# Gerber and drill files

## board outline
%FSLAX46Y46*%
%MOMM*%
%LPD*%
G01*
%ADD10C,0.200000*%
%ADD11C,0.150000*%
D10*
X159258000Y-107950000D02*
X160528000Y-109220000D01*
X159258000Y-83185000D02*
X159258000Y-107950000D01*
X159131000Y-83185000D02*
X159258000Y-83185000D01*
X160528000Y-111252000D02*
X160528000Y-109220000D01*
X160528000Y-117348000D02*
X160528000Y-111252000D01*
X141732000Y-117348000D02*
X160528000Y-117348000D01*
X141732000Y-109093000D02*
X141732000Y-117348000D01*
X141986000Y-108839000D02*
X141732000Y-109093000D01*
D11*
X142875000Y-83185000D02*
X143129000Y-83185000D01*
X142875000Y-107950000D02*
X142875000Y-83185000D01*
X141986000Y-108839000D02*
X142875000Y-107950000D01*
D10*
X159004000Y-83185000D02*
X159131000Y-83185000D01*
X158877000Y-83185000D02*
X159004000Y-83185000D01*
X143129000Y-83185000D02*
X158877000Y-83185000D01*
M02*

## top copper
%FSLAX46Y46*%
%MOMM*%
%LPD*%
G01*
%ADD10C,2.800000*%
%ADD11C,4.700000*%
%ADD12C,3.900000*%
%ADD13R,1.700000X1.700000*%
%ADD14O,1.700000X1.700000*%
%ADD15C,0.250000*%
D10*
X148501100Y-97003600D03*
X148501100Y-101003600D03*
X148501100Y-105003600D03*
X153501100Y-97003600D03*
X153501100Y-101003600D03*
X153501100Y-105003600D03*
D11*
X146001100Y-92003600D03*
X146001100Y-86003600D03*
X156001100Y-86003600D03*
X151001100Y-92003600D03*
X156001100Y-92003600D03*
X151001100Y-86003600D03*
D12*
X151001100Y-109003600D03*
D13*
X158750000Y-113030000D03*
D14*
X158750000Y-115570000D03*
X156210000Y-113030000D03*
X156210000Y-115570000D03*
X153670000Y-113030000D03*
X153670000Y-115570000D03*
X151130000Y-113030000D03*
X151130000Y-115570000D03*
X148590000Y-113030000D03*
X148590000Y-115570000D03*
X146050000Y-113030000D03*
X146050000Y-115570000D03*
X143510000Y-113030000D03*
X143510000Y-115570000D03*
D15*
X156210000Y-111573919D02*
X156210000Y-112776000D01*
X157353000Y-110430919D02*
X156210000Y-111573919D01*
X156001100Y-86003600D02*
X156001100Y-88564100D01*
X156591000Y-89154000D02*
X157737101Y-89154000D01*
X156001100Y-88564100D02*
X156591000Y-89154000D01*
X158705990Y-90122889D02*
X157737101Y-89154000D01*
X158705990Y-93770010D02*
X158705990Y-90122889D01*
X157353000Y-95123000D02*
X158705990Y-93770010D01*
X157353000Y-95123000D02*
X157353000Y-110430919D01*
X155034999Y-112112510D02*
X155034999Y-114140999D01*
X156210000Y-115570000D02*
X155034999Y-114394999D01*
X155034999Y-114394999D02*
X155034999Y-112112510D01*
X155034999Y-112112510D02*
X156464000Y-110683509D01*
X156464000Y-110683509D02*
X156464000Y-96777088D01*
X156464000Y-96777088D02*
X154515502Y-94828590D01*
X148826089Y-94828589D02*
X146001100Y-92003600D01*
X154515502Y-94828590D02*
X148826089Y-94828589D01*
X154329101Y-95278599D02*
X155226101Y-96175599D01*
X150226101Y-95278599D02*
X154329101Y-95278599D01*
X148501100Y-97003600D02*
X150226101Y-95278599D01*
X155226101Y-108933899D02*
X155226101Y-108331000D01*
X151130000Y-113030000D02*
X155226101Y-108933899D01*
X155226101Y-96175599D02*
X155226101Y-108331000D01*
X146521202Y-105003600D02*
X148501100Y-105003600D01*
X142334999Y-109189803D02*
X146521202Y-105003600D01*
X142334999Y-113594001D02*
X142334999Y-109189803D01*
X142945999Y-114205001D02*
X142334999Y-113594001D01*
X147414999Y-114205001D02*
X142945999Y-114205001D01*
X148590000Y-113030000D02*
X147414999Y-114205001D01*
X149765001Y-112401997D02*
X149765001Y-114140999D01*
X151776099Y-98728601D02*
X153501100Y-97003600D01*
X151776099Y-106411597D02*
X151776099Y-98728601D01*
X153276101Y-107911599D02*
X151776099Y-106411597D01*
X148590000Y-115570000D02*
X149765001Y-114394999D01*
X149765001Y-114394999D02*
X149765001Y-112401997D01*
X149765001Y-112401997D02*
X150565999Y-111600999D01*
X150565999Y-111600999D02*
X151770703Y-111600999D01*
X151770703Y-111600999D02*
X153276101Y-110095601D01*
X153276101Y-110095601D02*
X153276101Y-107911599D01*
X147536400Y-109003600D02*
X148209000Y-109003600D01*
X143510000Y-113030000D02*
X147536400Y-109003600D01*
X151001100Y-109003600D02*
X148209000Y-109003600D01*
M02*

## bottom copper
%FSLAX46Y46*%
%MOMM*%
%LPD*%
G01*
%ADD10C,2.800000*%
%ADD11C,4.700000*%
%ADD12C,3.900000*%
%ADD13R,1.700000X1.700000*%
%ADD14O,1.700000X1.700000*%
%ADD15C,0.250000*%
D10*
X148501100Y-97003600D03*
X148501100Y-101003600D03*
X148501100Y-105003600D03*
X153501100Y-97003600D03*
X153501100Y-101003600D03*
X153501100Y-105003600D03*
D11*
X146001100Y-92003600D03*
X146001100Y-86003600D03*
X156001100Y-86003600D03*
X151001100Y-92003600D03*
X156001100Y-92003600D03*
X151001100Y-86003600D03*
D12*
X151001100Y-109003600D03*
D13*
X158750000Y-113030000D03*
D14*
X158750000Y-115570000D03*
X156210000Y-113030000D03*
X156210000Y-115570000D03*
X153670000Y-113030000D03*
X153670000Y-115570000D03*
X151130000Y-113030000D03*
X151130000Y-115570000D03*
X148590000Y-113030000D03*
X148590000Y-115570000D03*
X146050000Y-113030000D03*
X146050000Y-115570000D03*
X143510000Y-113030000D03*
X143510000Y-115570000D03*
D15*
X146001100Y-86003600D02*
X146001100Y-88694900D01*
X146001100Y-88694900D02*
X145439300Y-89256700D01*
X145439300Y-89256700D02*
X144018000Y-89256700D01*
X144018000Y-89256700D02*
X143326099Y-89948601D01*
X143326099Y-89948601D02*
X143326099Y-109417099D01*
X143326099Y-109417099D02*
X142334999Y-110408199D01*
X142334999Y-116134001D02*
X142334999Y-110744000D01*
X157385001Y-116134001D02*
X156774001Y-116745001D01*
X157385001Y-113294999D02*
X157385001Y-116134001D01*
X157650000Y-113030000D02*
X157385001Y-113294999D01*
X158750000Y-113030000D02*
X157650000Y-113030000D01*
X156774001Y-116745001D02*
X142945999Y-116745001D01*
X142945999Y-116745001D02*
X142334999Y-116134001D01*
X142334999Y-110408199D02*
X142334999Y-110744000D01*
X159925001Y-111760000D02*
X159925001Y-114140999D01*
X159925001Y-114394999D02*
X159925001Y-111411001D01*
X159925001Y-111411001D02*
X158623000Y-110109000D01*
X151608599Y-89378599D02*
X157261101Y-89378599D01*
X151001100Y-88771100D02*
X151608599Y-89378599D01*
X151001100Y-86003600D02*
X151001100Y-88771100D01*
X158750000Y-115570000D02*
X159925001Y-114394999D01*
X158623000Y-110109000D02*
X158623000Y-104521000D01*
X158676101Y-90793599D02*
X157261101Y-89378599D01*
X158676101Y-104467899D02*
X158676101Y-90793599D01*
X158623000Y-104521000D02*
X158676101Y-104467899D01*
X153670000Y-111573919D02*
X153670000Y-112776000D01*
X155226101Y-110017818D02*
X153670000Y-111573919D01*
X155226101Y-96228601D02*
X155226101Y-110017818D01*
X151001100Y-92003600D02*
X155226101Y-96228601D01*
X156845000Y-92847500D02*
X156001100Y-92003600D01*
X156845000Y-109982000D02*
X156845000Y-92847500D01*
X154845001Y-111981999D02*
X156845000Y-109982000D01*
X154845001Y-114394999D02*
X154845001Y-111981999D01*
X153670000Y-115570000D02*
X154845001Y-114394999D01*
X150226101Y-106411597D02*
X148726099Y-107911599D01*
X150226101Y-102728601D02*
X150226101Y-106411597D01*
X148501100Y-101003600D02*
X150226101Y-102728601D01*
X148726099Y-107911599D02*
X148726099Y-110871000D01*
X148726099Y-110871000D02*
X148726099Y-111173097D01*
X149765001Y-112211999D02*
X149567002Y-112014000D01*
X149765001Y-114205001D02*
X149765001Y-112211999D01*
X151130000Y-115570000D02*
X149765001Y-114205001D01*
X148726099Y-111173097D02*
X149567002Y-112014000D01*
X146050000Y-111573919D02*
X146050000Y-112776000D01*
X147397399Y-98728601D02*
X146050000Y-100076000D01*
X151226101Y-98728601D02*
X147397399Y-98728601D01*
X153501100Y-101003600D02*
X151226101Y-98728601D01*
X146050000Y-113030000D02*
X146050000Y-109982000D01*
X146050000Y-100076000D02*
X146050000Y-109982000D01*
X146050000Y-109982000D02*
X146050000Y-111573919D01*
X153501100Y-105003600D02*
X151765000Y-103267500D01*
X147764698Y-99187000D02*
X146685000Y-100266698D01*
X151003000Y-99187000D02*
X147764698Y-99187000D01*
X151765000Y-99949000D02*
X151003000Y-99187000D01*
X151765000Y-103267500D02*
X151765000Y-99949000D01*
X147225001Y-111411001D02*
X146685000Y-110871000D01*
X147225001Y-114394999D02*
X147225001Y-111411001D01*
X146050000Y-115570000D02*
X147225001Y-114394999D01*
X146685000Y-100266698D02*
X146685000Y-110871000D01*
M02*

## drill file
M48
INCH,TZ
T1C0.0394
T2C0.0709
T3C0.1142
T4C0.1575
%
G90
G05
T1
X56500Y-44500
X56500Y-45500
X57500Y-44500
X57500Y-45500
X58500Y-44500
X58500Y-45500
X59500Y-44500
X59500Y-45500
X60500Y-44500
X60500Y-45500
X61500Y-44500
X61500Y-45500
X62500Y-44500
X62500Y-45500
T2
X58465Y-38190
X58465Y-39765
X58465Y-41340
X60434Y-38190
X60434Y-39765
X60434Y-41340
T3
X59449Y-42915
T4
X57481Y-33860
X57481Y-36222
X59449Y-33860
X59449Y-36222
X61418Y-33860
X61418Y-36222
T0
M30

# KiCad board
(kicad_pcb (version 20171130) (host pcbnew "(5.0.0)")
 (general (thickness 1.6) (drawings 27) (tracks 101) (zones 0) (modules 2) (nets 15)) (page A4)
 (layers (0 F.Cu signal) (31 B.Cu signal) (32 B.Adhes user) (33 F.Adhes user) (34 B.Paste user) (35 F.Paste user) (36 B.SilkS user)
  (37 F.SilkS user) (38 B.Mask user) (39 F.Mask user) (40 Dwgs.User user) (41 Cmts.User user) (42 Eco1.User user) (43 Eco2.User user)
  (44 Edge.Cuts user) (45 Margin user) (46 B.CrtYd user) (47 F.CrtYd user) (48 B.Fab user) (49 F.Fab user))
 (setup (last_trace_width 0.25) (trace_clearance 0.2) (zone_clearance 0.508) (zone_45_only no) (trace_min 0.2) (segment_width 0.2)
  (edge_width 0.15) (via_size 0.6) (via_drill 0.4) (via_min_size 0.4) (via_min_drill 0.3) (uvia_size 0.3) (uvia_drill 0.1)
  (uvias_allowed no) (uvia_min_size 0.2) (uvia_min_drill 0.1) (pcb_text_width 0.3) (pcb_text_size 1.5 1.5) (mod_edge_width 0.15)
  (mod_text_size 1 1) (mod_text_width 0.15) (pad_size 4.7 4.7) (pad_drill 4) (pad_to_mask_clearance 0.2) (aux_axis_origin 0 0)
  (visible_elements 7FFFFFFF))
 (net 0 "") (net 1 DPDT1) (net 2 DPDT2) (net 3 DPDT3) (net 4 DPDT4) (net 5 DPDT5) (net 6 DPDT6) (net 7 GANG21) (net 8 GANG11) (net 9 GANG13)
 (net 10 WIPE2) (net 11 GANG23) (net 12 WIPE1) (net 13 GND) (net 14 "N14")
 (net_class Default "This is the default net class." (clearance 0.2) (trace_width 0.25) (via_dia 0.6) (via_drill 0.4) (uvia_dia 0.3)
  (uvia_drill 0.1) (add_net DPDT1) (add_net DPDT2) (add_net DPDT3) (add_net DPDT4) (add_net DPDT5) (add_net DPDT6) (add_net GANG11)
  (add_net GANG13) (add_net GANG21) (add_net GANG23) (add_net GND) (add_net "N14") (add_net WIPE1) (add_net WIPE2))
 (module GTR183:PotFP (layer F.Cu) (at 148.5011 105.0036)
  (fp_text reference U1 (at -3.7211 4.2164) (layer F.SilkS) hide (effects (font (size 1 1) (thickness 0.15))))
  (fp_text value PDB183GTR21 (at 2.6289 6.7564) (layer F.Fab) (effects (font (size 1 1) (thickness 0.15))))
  (pad 7 thru_hole circle (at 0 -8) (size 2.8 2.8) (drill 1.8) (layers *.Cu *.Mask F.SilkS) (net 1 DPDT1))
  (pad 8 thru_hole circle (at 0 -4) (size 2.8 2.8) (drill 1.8) (layers *.Cu *.Mask F.SilkS) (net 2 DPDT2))
  (pad 9 thru_hole circle (at 0 0) (size 2.8 2.8) (drill 1.8) (layers *.Cu *.Mask F.SilkS) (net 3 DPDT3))
  (pad 10 thru_hole circle (at 5 -8) (size 2.8 2.8) (drill 1.8) (layers *.Cu *.Mask F.SilkS) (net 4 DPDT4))
  (pad 11 thru_hole circle (at 5 -4) (size 2.8 2.8) (drill 1.8) (layers *.Cu *.Mask F.SilkS) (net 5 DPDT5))
  (pad 12 thru_hole circle (at 5 0) (size 2.8 2.8) (drill 1.8) (layers *.Cu *.Mask F.SilkS) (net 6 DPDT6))
  (pad 4 thru_hole circle (at -2.5 -13) (size 4.7 4.7) (drill 4) (layers *.Cu *.Mask F.SilkS) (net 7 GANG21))
  (pad 1 thru_hole circle (at -2.5 -19) (size 4.7 4.7) (drill 4) (layers *.Cu *.Mask F.SilkS) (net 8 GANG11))
  (pad 3 thru_hole circle (at 7.5 -19) (size 4.7 4.7) (drill 4) (layers *.Cu *.Mask F.SilkS) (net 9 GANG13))
  (pad 5 thru_hole circle (at 2.5 -13) (size 4.7 4.7) (drill 4) (layers *.Cu *.Mask F.SilkS) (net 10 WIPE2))
  (pad 6 thru_hole circle (at 7.5 -13) (size 4.7 4.7) (drill 4) (layers *.Cu *.Mask F.SilkS) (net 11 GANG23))
  (pad 2 thru_hole circle (at 2.5 -19) (size 4.7 4.7) (drill 4) (layers *.Cu *.Mask F.SilkS) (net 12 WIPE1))
  (pad 13 thru_hole circle (at 2.5 4) (size 3.9 3.9) (drill 2.9) (layers *.Cu *.Mask F.SilkS) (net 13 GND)))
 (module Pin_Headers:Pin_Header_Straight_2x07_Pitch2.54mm (layer F.Cu) (at 158.75 113.03 270)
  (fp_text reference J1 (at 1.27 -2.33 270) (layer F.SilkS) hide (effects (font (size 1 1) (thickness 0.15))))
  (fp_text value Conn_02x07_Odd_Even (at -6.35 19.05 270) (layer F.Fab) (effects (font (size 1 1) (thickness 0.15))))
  (pad 1 thru_hole rect (at 0 0 270) (size 1.7 1.7) (drill 1) (layers *.Cu *.Mask) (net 8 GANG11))
  (pad 2 thru_hole oval (at 2.54 0 270) (size 1.7 1.7) (drill 1) (layers *.Cu *.Mask) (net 12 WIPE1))
  (pad 3 thru_hole oval (at 0 2.54 270) (size 1.7 1.7) (drill 1) (layers *.Cu *.Mask) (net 9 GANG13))
  (pad 4 thru_hole oval (at 2.54 2.54 270) (size 1.7 1.7) (drill 1) (layers *.Cu *.Mask) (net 7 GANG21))
  (pad 5 thru_hole oval (at 0 5.08 270) (size 1.7 1.7) (drill 1) (layers *.Cu *.Mask) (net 10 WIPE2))
  (pad 6 thru_hole oval (at 2.54 5.08 270) (size 1.7 1.7) (drill 1) (layers *.Cu *.Mask) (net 11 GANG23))
  (pad 7 thru_hole oval (at 0 7.62 270) (size 1.7 1.7) (drill 1) (layers *.Cu *.Mask) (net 1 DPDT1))
  (pad 8 thru_hole oval (at 2.54 7.62 270) (size 1.7 1.7) (drill 1) (layers *.Cu *.Mask) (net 2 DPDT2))
  (pad 9 thru_hole oval (at 0 10.16 270) (size 1.7 1.7) (drill 1) (layers *.Cu *.Mask) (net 3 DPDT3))
  (pad 10 thru_hole oval (at 2.54 10.16 270) (size 1.7 1.7) (drill 1) (layers *.Cu *.Mask) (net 4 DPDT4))
  (pad 11 thru_hole oval (at 0 12.7 270) (size 1.7 1.7) (drill 1) (layers *.Cu *.Mask) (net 5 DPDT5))
  (pad 12 thru_hole oval (at 2.54 12.7 270) (size 1.7 1.7) (drill 1) (layers *.Cu *.Mask) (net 6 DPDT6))
  (pad 13 thru_hole oval (at 0 15.24 270) (size 1.7 1.7) (drill 1) (layers *.Cu *.Mask) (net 13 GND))
  (pad 14 thru_hole oval (at 2.54 15.24 270) (size 1.7 1.7) (drill 1) (layers *.Cu *.Mask) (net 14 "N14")))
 (gr_line (start 159.258 107.95) (end 160.528 109.22) (layer Edge.Cuts) (width 0.2))
 (gr_line (start 159.258 83.185) (end 159.258 107.95) (layer Edge.Cuts) (width 0.2))
 (gr_line (start 159.131 83.185) (end 159.258 83.185) (layer Edge.Cuts) (width 0.2))
 (gr_line (start 160.528 111.252) (end 160.528 109.22) (layer Edge.Cuts) (width 0.2))
 (gr_line (start 160.528 117.348) (end 160.528 111.252) (layer Edge.Cuts) (width 0.2))
 (gr_line (start 141.732 117.348) (end 160.528 117.348) (layer Edge.Cuts) (width 0.2))
 (gr_line (start 141.732 109.093) (end 141.732 117.348) (layer Edge.Cuts) (width 0.2))
 (gr_line (start 141.986 108.839) (end 141.732 109.093) (layer Edge.Cuts) (width 0.2))
 (gr_line (start 142.875 83.185) (end 143.129 83.185) (layer Edge.Cuts) (width 0.15))
 (gr_line (start 142.875 107.95) (end 142.875 83.185) (layer Edge.Cuts) (width 0.15))
 (gr_line (start 141.986 108.839) (end 142.875 107.95) (layer Edge.Cuts) (width 0.15))
 (gr_line (start 159.004 83.185) (end 159.131 83.185) (layer Edge.Cuts) (width 0.2))
 (gr_line (start 158.877 83.185) (end 159.004 83.185) (layer Edge.Cuts) (width 0.2))
 (gr_line (start 143.129 83.185) (end 158.877 83.185) (layer Edge.Cuts) (width 0.2))
 (segment (start 146.0011 86.0036) (end 146.0011 88.6949) (width 0.25) (layer B.Cu) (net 8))
 (segment (start 146.0011 88.6949) (end 145.4393 89.2567) (width 0.25) (layer B.Cu) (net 8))
 (segment (start 145.4393 89.2567) (end 144.018 89.2567) (width 0.25) (layer B.Cu) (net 8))
 (segment (start 144.018 89.2567) (end 143.326099 89.948601) (width 0.25) (layer B.Cu) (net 8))
 (segment (start 143.326099 89.948601) (end 143.326099 109.417099) (width 0.25) (layer B.Cu) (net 8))
 (segment (start 143.326099 109.417099) (end 142.334999 110.408199) (width 0.25) (layer B.Cu) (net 8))
 (segment (start 142.334999 116.134001) (end 142.334999 110.744) (width 0.25) (layer B.Cu) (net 8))
 (segment (start 157.385001 116.134001) (end 156.774001 116.745001) (width 0.25) (layer B.Cu) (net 8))
 (segment (start 157.385001 113.294999) (end 157.385001 116.134001) (width 0.25) (layer B.Cu) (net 8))
 (segment (start 157.65 113.03) (end 157.385001 113.294999) (width 0.25) (layer B.Cu) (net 8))
 (segment (start 158.75 113.03) (end 157.65 113.03) (width 0.25) (layer B.Cu) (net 8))
 (segment (start 156.774001 116.745001) (end 142.945999 116.745001) (width 0.25) (layer B.Cu) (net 8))
 (segment (start 142.945999 116.745001) (end 142.334999 116.134001) (width 0.25) (layer B.Cu) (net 8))
 (segment (start 142.334999 110.408199) (end 142.334999 110.744) (width 0.25) (layer B.Cu) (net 8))
 (segment (start 159.925001 111.76) (end 159.925001 114.140999) (width 0.25) (layer B.Cu) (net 12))
 (segment (start 159.925001 114.394999) (end 159.925001 111.411001) (width 0.25) (layer B.Cu) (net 12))
 (segment (start 159.925001 111.411001) (end 158.623 110.109) (width 0.25) (layer B.Cu) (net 12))
 (segment (start 151.608599 89.378599) (end 157.261101 89.378599) (width 0.25) (layer B.Cu) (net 12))
 (segment (start 151.0011 88.7711) (end 151.608599 89.378599) (width 0.25) (layer B.Cu) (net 12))
 (segment (start 151.0011 86.0036) (end 151.0011 88.7711) (width 0.25) (layer B.Cu) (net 12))
 (segment (start 158.75 115.57) (end 159.925001 114.394999) (width 0.25) (layer B.Cu) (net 12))
 (segment (start 158.623 110.109) (end 158.623 104.521) (width 0.25) (layer B.Cu) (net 12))
 (segment (start 158.676101 90.793599) (end 157.261101 89.378599) (width 0.25) (layer B.Cu) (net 12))
 (segment (start 158.676101 104.467899) (end 158.676101 90.793599) (width 0.25) (layer B.Cu) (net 12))
 (segment (start 158.623 104.521) (end 158.676101 104.467899) (width 0.25) (layer B.Cu) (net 12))
 (segment (start 156.21 111.573919) (end 156.21 112.776) (width 0.25) (layer F.Cu) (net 9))
 (segment (start 157.353 110.430919) (end 156.21 111.573919) (width 0.25) (layer F.Cu) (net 9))
 (segment (start 156.0011 86.0036) (end 156.0011 88.5641) (width 0.25) (layer F.Cu) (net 9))
 (segment (start 156.591 89.154) (end 157.737101 89.154) (width 0.25) (layer F.Cu) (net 9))
 (segment (start 156.0011 88.5641) (end 156.591 89.154) (width 0.25) (layer F.Cu) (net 9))
 (segment (start 158.70599 90.122889) (end 157.737101 89.154) (width 0.25) (layer F.Cu) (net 9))
 (segment (start 158.70599 93.77001) (end 158.70599 90.122889) (width 0.25) (layer F.Cu) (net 9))
 (segment (start 157.353 95.123) (end 158.70599 93.77001) (width 0.25) (layer F.Cu) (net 9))
 (segment (start 157.353 95.123) (end 157.353 110.430919) (width 0.25) (layer F.Cu) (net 9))
 (segment (start 155.034999 112.11251) (end 155.034999 114.140999) (width 0.25) (layer F.Cu) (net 7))
 (segment (start 156.21 115.57) (end 155.034999 114.394999) (width 0.25) (layer F.Cu) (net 7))
 (segment (start 155.034999 114.394999) (end 155.034999 112.11251) (width 0.25) (layer F.Cu) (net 7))
 (segment (start 155.034999 112.11251) (end 156.464 110.683509) (width 0.25) (layer F.Cu) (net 7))
 (segment (start 156.464 110.683509) (end 156.464 96.777088) (width 0.25) (layer F.Cu) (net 7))
 (segment (start 156.464 96.777088) (end 154.515502 94.82859) (width 0.25) (layer F.Cu) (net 7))
 (segment (start 148.826089 94.828589) (end 146.0011 92.0036) (width 0.25) (layer F.Cu) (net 7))
 (segment (start 154.515502 94.82859) (end 148.826089 94.828589) (width 0.25) (layer F.Cu) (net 7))
 (segment (start 153.67 111.573919) (end 153.67 112.776) (width 0.25) (layer B.Cu) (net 10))
 (segment (start 155.226101 110.017818) (end 153.67 111.573919) (width 0.25) (layer B.Cu) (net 10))
 (segment (start 155.226101 96.228601) (end 155.226101 110.017818) (width 0.25) (layer B.Cu) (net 10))
 (segment (start 151.0011 92.0036) (end 155.226101 96.228601) (width 0.25) (layer B.Cu) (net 10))
 (segment (start 156.845 92.8475) (end 156.0011 92.0036) (width 0.25) (layer B.Cu) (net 11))
 (segment (start 156.845 109.982) (end 156.845 92.8475) (width 0.25) (layer B.Cu) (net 11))
 (segment (start 154.845001 111.981999) (end 156.845 109.982) (width 0.25) (layer B.Cu) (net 11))
 (segment (start 154.845001 114.394999) (end 154.845001 111.981999) (width 0.25) (layer B.Cu) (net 11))
 (segment (start 153.67 115.57) (end 154.845001 114.394999) (width 0.25) (layer B.Cu) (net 11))
 (segment (start 154.329101 95.278599) (end 155.226101 96.175599) (width 0.25) (layer F.Cu) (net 1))
 (segment (start 150.226101 95.278599) (end 154.329101 95.278599) (width 0.25) (layer F.Cu) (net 1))
 (segment (start 148.5011 97.0036) (end 150.226101 95.278599) (width 0.25) (layer F.Cu) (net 1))
 (segment (start 155.226101 108.933899) (end 155.226101 108.331) (width 0.25) (layer F.Cu) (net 1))
 (segment (start 151.13 113.03) (end 155.226101 108.933899) (width 0.25) (layer F.Cu) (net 1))
 (segment (start 155.226101 96.175599) (end 155.226101 108.331) (width 0.25) (layer F.Cu) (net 1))
 (segment (start 150.226101 106.411597) (end 148.726099 107.911599) (width 0.25) (layer B.Cu) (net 2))
 (segment (start 150.226101 102.728601) (end 150.226101 106.411597) (width 0.25) (layer B.Cu) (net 2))
 (segment (start 148.5011 101.0036) (end 150.226101 102.728601) (width 0.25) (layer B.Cu) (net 2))
 (segment (start 148.726099 107.911599) (end 148.726099 110.871) (width 0.25) (layer B.Cu) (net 2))
 (segment (start 148.726099 110.871) (end 148.726099 111.173097) (width 0.25) (layer B.Cu) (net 2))
 (segment (start 149.765001 112.211999) (end 149.567002 112.014) (width 0.25) (layer B.Cu) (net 2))
 (segment (start 149.765001 114.205001) (end 149.765001 112.211999) (width 0.25) (layer B.Cu) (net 2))
 (segment (start 151.13 115.57) (end 149.765001 114.205001) (width 0.25) (layer B.Cu) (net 2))
 (segment (start 148.726099 111.173097) (end 149.567002 112.014) (width 0.25) (layer B.Cu) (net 2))
 (segment (start 146.521202 105.0036) (end 148.5011 105.0036) (width 0.25) (layer F.Cu) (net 3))
 (segment (start 142.334999 109.189803) (end 146.521202 105.0036) (width 0.25) (layer F.Cu) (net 3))
 (segment (start 142.334999 113.594001) (end 142.334999 109.189803) (width 0.25) (layer F.Cu) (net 3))
 (segment (start 142.945999 114.205001) (end 142.334999 113.594001) (width 0.25) (layer F.Cu) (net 3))
 (segment (start 147.414999 114.205001) (end 142.945999 114.205001) (width 0.25) (layer F.Cu) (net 3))
 (segment (start 148.59 113.03) (end 147.414999 114.205001) (width 0.25) (layer F.Cu) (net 3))
 (segment (start 149.765001 112.401997) (end 149.765001 114.140999) (width 0.25) (layer F.Cu) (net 4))
 (segment (start 151.776099 98.728601) (end 153.5011 97.0036) (width 0.25) (layer F.Cu) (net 4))
 (segment (start 151.776099 106.411597) (end 151.776099 98.728601) (width 0.25) (layer F.Cu) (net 4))
 (segment (start 153.276101 107.911599) (end 151.776099 106.411597) (width 0.25) (layer F.Cu) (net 4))
 (segment (start 148.59 115.57) (end 149.765001 114.394999) (width 0.25) (layer F.Cu) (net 4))
 (segment (start 149.765001 114.394999) (end 149.765001 112.401997) (width 0.25) (layer F.Cu) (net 4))
 (segment (start 149.765001 112.401997) (end 150.565999 111.600999) (width 0.25) (layer F.Cu) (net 4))
 (segment (start 150.565999 111.600999) (end 151.770703 111.600999) (width 0.25) (layer F.Cu) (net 4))
 (segment (start 151.770703 111.600999) (end 153.276101 110.095601) (width 0.25) (layer F.Cu) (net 4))
 (segment (start 153.276101 110.095601) (end 153.276101 107.911599) (width 0.25) (layer F.Cu) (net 4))
 (segment (start 146.05 111.573919) (end 146.05 112.776) (width 0.25) (layer B.Cu) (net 5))
 (segment (start 147.397399 98.728601) (end 146.05 100.076) (width 0.25) (layer B.Cu) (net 5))
 (segment (start 151.226101 98.728601) (end 147.397399 98.728601) (width 0.25) (layer B.Cu) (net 5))
 (segment (start 153.5011 101.0036) (end 151.226101 98.728601) (width 0.25) (layer B.Cu) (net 5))
 (segment (start 146.05 113.03) (end 146.05 109.982) (width 0.25) (layer B.Cu) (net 5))
 (segment (start 146.05 100.076) (end 146.05 109.982) (width 0.25) (layer B.Cu) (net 5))
 (segment (start 146.05 109.982) (end 146.05 111.573919) (width 0.25) (layer B.Cu) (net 5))
 (segment (start 153.5011 105.0036) (end 151.765 103.2675) (width 0.25) (layer B.Cu) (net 6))
 (segment (start 147.764698 99.187) (end 146.685 100.266698) (width 0.25) (layer B.Cu) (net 6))
 (segment (start 151.003 99.187) (end 147.764698 99.187) (width 0.25) (layer B.Cu) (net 6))
 (segment (start 151.765 99.949) (end 151.003 99.187) (width 0.25) (layer B.Cu) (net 6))
 (segment (start 151.765 103.2675) (end 151.765 99.949) (width 0.25) (layer B.Cu) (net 6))
 (segment (start 147.225001 111.411001) (end 146.685 110.871) (width 0.25) (layer B.Cu) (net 6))
 (segment (start 147.225001 114.394999) (end 147.225001 111.411001) (width 0.25) (layer B.Cu) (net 6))
 (segment (start 146.05 115.57) (end 147.225001 114.394999) (width 0.25) (layer B.Cu) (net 6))
 (segment (start 146.685 100.266698) (end 146.685 110.871) (width 0.25) (layer B.Cu) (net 6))
 (segment (start 147.5364 109.0036) (end 148.209 109.0036) (width 0.25) (layer F.Cu) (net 13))
 (segment (start 143.51 113.03) (end 147.5364 109.0036) (width 0.25) (layer F.Cu) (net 13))
 (segment (start 151.0011 109.0036) (end 148.209 109.0036) (width 0.25) (layer F.Cu) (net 13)))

